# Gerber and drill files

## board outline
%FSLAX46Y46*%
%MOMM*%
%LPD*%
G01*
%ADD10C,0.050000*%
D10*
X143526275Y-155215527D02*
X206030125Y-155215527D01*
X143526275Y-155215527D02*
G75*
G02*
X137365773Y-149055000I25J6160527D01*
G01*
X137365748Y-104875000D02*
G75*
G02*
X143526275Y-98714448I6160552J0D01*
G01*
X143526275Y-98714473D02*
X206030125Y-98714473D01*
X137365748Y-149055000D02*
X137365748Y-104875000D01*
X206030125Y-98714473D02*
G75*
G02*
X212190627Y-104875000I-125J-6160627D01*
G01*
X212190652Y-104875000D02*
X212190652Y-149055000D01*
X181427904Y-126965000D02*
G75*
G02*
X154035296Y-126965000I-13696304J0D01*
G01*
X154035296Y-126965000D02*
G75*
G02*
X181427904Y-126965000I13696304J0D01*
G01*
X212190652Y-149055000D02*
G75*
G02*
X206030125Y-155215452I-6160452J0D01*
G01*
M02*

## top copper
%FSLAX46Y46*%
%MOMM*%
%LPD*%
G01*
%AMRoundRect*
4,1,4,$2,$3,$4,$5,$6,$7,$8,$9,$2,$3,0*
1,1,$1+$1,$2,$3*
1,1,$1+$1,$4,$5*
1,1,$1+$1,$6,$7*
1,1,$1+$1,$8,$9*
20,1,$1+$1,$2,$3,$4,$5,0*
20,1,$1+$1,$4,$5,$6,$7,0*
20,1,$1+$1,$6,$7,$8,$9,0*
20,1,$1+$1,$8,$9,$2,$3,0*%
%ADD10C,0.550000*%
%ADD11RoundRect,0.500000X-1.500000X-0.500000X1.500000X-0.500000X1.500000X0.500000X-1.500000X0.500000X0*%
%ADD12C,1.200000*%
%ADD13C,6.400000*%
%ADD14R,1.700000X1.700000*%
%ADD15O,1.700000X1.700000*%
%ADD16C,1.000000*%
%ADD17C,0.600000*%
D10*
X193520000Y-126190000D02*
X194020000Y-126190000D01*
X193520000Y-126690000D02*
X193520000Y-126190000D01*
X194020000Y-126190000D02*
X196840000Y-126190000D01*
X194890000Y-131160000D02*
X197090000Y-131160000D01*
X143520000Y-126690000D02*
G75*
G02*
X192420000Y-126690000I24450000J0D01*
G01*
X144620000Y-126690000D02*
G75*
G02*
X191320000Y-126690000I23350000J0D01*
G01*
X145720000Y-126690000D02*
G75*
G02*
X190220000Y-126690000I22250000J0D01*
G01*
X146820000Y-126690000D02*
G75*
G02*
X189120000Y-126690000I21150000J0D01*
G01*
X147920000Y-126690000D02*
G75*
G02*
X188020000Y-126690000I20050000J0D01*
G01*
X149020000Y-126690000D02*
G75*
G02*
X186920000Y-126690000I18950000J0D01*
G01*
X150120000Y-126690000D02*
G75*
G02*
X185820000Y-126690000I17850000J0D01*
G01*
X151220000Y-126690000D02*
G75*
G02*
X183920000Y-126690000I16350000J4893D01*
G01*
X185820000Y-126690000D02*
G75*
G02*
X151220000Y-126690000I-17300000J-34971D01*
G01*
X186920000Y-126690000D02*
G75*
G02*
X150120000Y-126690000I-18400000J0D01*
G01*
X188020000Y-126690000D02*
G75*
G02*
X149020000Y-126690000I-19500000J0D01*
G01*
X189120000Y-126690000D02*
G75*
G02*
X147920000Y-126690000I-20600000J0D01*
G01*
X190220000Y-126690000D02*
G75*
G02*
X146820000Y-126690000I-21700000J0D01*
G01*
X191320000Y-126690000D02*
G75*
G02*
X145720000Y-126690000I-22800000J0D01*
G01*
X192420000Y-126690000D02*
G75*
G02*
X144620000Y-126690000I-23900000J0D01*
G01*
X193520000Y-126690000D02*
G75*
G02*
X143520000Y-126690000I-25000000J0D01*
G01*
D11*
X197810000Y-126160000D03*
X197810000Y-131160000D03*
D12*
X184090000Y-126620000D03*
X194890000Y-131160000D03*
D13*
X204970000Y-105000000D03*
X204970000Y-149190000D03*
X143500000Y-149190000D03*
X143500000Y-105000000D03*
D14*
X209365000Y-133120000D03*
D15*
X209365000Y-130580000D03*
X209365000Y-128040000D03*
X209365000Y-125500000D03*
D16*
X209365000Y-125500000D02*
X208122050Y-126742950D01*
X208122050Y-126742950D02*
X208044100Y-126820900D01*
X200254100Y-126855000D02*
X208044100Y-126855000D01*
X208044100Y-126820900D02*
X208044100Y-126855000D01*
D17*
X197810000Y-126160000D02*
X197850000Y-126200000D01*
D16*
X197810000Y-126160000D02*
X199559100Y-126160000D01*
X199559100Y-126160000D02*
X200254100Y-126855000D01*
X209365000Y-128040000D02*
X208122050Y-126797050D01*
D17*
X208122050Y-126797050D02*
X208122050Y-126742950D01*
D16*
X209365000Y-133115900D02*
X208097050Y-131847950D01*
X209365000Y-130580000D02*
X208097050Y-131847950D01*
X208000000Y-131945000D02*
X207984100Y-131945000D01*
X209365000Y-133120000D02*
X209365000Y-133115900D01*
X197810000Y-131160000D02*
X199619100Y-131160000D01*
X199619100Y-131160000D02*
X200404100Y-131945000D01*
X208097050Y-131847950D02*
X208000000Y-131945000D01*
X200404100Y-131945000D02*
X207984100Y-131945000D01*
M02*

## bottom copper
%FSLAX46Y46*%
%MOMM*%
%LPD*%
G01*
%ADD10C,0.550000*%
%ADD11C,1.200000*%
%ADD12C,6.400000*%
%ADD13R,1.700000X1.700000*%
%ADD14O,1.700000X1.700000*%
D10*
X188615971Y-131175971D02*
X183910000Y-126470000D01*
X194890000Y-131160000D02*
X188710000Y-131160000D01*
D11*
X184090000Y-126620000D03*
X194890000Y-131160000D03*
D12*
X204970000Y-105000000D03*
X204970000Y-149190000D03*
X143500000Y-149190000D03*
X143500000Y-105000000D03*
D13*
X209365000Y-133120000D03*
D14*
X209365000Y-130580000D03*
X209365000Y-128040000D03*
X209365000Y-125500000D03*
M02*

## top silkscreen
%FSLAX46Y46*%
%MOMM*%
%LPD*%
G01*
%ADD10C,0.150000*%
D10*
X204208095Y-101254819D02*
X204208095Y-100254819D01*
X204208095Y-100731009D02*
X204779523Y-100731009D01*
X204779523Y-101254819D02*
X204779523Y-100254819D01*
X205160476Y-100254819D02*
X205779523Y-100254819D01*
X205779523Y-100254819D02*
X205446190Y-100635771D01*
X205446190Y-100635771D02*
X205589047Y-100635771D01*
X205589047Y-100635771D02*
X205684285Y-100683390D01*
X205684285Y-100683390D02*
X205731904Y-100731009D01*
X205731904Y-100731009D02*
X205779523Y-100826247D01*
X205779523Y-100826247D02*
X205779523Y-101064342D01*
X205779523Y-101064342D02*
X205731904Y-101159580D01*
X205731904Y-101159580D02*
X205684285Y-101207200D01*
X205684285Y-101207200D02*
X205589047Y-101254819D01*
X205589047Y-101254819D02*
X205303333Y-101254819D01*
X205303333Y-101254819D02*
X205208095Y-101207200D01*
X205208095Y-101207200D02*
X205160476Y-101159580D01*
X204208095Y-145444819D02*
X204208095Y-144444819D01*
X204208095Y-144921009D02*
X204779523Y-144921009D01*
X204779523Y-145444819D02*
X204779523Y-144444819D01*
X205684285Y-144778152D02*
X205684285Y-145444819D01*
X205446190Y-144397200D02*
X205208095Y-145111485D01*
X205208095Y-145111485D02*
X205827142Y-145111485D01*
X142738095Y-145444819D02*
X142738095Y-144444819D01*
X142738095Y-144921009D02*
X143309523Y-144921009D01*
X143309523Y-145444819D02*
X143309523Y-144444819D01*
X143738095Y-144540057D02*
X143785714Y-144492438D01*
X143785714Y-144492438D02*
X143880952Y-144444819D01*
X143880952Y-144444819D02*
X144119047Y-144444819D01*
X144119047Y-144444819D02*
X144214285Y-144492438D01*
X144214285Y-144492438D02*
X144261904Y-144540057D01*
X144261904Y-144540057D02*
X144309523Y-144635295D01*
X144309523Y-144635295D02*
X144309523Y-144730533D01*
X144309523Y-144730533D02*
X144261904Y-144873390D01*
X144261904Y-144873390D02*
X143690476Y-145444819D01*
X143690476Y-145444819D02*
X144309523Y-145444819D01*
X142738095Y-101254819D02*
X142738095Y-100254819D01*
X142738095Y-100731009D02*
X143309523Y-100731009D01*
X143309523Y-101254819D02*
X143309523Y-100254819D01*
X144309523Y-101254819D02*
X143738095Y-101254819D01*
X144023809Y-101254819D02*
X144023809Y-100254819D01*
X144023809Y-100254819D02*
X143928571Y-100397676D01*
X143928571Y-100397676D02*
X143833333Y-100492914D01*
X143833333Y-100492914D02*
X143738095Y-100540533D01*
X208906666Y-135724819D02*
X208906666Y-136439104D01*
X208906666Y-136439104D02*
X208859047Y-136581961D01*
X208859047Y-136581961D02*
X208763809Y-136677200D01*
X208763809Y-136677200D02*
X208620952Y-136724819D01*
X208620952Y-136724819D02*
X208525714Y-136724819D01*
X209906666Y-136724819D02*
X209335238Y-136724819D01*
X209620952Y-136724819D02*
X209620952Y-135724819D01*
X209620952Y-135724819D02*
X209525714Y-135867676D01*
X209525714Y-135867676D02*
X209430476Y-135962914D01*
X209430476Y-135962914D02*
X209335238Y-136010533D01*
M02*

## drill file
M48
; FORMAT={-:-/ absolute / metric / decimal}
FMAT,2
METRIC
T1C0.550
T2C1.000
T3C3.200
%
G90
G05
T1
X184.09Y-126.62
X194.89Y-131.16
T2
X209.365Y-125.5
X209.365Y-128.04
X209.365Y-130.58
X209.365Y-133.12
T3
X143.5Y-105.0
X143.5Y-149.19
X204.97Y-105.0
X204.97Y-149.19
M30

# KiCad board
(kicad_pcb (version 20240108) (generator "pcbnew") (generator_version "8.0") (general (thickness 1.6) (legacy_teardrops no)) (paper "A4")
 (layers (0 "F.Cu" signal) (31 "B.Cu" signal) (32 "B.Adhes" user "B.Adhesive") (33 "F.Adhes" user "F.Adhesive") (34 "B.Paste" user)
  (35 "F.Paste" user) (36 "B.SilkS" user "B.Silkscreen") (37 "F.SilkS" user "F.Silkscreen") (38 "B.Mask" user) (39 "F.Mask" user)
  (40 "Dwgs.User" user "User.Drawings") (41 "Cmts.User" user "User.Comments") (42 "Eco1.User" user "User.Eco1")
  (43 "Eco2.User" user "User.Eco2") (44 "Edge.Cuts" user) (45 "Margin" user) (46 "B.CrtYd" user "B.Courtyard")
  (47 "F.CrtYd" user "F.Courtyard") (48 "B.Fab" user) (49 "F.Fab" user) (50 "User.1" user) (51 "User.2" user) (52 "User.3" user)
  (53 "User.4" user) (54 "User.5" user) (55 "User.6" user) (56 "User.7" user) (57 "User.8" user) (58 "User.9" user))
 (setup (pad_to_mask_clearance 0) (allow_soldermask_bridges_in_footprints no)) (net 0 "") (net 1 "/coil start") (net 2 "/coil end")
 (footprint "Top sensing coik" (layer "F.Cu") (at 167.97 126.69)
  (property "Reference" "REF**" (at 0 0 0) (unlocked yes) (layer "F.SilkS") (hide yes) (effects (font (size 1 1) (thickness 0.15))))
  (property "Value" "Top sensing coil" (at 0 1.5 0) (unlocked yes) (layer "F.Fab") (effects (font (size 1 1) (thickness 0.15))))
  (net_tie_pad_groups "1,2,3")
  (fp_line (start 25.55 -0.5) (end 26.05 -0.5) (stroke (width 0.55) (type solid)) (layer "F.Cu"))
  (fp_line (start 25.55 0) (end 25.55 -0.5) (stroke (width 0.55) (type solid)) (layer "F.Cu"))
  (fp_line (start 26.05 -0.5) (end 28.87 -0.5) (stroke (width 0.55) (type default)) (layer "F.Cu"))
  (fp_line (start 26.92 4.47) (end 29.12 4.47) (stroke (width 0.55) (type default)) (layer "F.Cu"))
  (fp_arc (start -24.45 0) (mid 0 -24.45) (end 24.45 0) (stroke (width 0.55) (type solid)) (layer "F.Cu"))
  (fp_arc (start -23.35 0) (mid 0 -23.35) (end 23.35 0) (stroke (width 0.55) (type solid)) (layer "F.Cu"))
  (fp_arc (start -22.25 0) (mid 0 -22.25) (end 22.25 0) (stroke (width 0.55) (type solid)) (layer "F.Cu"))
  (fp_arc (start -21.15 0) (mid 0 -21.15) (end 21.15 0) (stroke (width 0.55) (type solid)) (layer "F.Cu"))
  (fp_arc (start -20.05 0) (mid 0 -20.05) (end 20.05 0) (stroke (width 0.55) (type solid)) (layer "F.Cu"))
  (fp_arc (start -18.95 0) (mid 0 -18.95) (end 18.95 0) (stroke (width 0.55) (type solid)) (layer "F.Cu"))
  (fp_arc (start -17.85 0) (mid 0 -17.85) (end 17.85 0) (stroke (width 0.55) (type solid)) (layer "F.Cu"))
  (fp_arc (start -16.75 0) (mid -0.4 -16.354894) (end 15.95 0) (stroke (width 0.55) (type solid)) (layer "F.Cu"))
  (fp_arc (start 17.85 0) (mid 0.55 17.335006) (end -16.75 0) (stroke (width 0.55) (type solid)) (layer "F.Cu"))
  (fp_arc (start 18.95 0) (mid 0.55 18.4) (end -17.85 0) (stroke (width 0.55) (type solid)) (layer "F.Cu"))
  (fp_arc (start 20.05 0) (mid 0.55 19.5) (end -18.95 0) (stroke (width 0.55) (type solid)) (layer "F.Cu"))
  (fp_arc (start 21.15 0) (mid 0.55 20.6) (end -20.05 0) (stroke (width 0.55) (type solid)) (layer "F.Cu"))
  (fp_arc (start 22.25 0) (mid 0.55 21.7) (end -21.15 0) (stroke (width 0.55) (type solid)) (layer "F.Cu"))
  (fp_arc (start 23.35 0) (mid 0.55 22.8) (end -22.25 0) (stroke (width 0.55) (type solid)) (layer "F.Cu"))
  (fp_arc (start 24.45 0) (mid 0.55 23.9) (end -23.35 0) (stroke (width 0.55) (type solid)) (layer "F.Cu"))
  (fp_arc (start 25.55 0) (mid 0.55 25) (end -24.45 0) (stroke (width 0.55) (type solid)) (layer "F.Cu"))
  (fp_line (start 20.645971 4.485971) (end 15.94 -0.22) (stroke (width 0.55) (type default)) (layer "B.Cu"))
  (fp_line (start 26.92 4.47) (end 20.74 4.47) (stroke (width 0.55) (type default)) (layer "B.Cu"))
  (pad "1" smd roundrect (at 29.84 -0.53) (size 4 2) (layers "F.Cu") (roundrect_rratio 0.25) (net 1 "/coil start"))
  (pad "2" smd roundrect (at 29.84 4.47) (size 4 2) (layers "F.Cu") (roundrect_rratio 0.25) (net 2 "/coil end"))
  (pad "3" thru_hole circle (at 16.12 -0.07 90) (size 1.2 1.2) (drill 0.55) (layers "*.Cu" "*.Mask") (remove_unused_layers no))
  (pad "3" thru_hole circle (at 26.92 4.47 90) (size 1.2 1.2) (drill 0.55) (layers "*.Cu" "*.Mask") (remove_unused_layers no)))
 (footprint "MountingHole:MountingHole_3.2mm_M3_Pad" (layer "F.Cu") (at 204.97 105)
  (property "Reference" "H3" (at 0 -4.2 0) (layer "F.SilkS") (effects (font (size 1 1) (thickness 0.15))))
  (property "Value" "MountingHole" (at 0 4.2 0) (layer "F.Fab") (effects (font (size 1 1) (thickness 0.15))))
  (pad "1" thru_hole circle (at 0 0) (size 6.4 6.4) (drill 3.2) (layers "*.Cu" "*.Mask") (remove_unused_layers no)))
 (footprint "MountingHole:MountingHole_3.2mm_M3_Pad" (layer "F.Cu") (at 204.97 149.19)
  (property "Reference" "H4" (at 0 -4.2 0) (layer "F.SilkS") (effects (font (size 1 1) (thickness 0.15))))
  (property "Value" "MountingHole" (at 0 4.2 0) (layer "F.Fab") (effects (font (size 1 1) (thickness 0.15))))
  (pad "1" thru_hole circle (at 0 0) (size 6.4 6.4) (drill 3.2) (layers "*.Cu" "*.Mask") (remove_unused_layers no)))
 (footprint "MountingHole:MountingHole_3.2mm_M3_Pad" (layer "F.Cu") (at 143.5 149.19)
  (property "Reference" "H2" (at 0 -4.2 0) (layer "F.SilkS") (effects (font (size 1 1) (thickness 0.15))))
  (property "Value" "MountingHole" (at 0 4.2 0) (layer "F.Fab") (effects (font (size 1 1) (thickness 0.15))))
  (pad "1" thru_hole circle (at 0 0) (size 6.4 6.4) (drill 3.2) (layers "*.Cu" "*.Mask") (remove_unused_layers no)))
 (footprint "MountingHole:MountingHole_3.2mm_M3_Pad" (layer "F.Cu") (at 143.5 105)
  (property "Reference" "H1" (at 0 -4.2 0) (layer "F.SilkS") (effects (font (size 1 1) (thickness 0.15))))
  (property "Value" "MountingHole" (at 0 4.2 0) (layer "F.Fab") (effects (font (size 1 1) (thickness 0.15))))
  (pad "1" thru_hole circle (at 0 0) (size 6.4 6.4) (drill 3.2) (layers "*.Cu" "*.Mask") (remove_unused_layers no)))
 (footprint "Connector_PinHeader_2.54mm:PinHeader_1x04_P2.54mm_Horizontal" (layer "B.Cu") (at 209.365 133.12)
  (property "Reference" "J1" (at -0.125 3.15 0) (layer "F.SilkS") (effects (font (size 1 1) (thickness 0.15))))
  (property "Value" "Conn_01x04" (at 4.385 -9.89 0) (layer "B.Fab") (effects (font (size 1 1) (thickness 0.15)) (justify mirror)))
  (pad "1" thru_hole rect (at 0 0) (size 1.7 1.7) (drill 1) (layers "*.Cu" "*.Mask") (remove_unused_layers no) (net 2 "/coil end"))
  (pad "2" thru_hole oval (at 0 -2.54) (size 1.7 1.7) (drill 1) (layers "*.Cu" "*.Mask") (remove_unused_layers no) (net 2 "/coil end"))
  (pad "3" thru_hole oval (at 0 -5.08) (size 1.7 1.7) (drill 1) (layers "*.Cu" "*.Mask") (remove_unused_layers no) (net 1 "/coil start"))
  (pad "4" thru_hole oval (at 0 -7.62) (size 1.7 1.7) (drill 1) (layers "*.Cu" "*.Mask") (remove_unused_layers no) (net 1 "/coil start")))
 (gr_line (start 143.526275 155.215527) (end 206.030125 155.215527) (stroke (width 0.05) (type default)) (layer "Edge.Cuts"))
 (gr_arc (start 143.526275 155.215527) (mid 139.170125 153.41115) (end 137.365748 149.055) (stroke (width 0.05) (type default))
  (layer "Edge.Cuts"))
 (gr_arc (start 137.365748 104.875) (mid 139.170125 100.51885) (end 143.526275 98.714473) (stroke (width 0.05) (type default))
  (layer "Edge.Cuts"))
 (gr_line (start 143.526275 98.714473) (end 206.030125 98.714473) (stroke (width 0.05) (type default)) (layer "Edge.Cuts"))
 (gr_line (start 137.365748 149.055) (end 137.365748 104.875) (stroke (width 0.05) (type default)) (layer "Edge.Cuts"))
 (gr_arc (start 206.030125 98.714473) (mid 210.386228 100.518882) (end 212.190652 104.875) (stroke (width 0.05) (type default))
  (layer "Edge.Cuts"))
 (gr_line (start 212.190652 104.875) (end 212.190652 149.055) (stroke (width 0.05) (type default)) (layer "Edge.Cuts"))
 (gr_circle (center 167.7316 126.965) (end 179.97 120.815992) (stroke (width 0.05) (type default)) (fill none) (layer "Edge.Cuts"))
 (gr_arc (start 212.190652 149.055) (mid 210.386284 153.411159) (end 206.030125 155.215527) (stroke (width 0.05) (type default))
  (layer "Edge.Cuts"))
 (segment (start 209.365 125.5) (end 208.12205 126.74295) (width 1) (layer "F.Cu") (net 1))
 (segment (start 208.12205 126.74295) (end 208.0441 126.8209) (width 1) (layer "F.Cu") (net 1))
 (segment (start 200.2541 126.855) (end 208.0441 126.855) (width 1) (layer "F.Cu") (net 1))
 (segment (start 208.0441 126.8209) (end 208.0441 126.855) (width 1) (layer "F.Cu") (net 1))
 (segment (start 197.81 126.16) (end 197.85 126.2) (width 0.6) (layer "F.Cu") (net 1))
 (segment (start 197.81 126.16) (end 199.5591 126.16) (width 1) (layer "F.Cu") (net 1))
 (segment (start 199.5591 126.16) (end 200.2541 126.855) (width 1) (layer "F.Cu") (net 1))
 (segment (start 209.365 128.04) (end 208.12205 126.79705) (width 1) (layer "F.Cu") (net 1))
 (segment (start 208.12205 126.79705) (end 208.12205 126.74295) (width 0.6) (layer "F.Cu") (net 1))
 (segment (start 209.365 133.1159) (end 208.09705 131.84795) (width 1) (layer "F.Cu") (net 2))
 (segment (start 209.365 130.58) (end 208.09705 131.84795) (width 1) (layer "F.Cu") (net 2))
 (segment (start 208 131.945) (end 207.9841 131.945) (width 1) (layer "F.Cu") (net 2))
 (segment (start 209.365 133.12) (end 209.365 133.1159) (width 1) (layer "F.Cu") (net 2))
 (segment (start 197.81 131.16) (end 199.6191 131.16) (width 1) (layer "F.Cu") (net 2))
 (segment (start 199.6191 131.16) (end 200.4041 131.945) (width 1) (layer "F.Cu") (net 2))
 (segment (start 208.09705 131.84795) (end 208 131.945) (width 1) (layer "F.Cu") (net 2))
 (segment (start 200.4041 131.945) (end 207.9841 131.945) (width 1) (layer "F.Cu") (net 2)))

